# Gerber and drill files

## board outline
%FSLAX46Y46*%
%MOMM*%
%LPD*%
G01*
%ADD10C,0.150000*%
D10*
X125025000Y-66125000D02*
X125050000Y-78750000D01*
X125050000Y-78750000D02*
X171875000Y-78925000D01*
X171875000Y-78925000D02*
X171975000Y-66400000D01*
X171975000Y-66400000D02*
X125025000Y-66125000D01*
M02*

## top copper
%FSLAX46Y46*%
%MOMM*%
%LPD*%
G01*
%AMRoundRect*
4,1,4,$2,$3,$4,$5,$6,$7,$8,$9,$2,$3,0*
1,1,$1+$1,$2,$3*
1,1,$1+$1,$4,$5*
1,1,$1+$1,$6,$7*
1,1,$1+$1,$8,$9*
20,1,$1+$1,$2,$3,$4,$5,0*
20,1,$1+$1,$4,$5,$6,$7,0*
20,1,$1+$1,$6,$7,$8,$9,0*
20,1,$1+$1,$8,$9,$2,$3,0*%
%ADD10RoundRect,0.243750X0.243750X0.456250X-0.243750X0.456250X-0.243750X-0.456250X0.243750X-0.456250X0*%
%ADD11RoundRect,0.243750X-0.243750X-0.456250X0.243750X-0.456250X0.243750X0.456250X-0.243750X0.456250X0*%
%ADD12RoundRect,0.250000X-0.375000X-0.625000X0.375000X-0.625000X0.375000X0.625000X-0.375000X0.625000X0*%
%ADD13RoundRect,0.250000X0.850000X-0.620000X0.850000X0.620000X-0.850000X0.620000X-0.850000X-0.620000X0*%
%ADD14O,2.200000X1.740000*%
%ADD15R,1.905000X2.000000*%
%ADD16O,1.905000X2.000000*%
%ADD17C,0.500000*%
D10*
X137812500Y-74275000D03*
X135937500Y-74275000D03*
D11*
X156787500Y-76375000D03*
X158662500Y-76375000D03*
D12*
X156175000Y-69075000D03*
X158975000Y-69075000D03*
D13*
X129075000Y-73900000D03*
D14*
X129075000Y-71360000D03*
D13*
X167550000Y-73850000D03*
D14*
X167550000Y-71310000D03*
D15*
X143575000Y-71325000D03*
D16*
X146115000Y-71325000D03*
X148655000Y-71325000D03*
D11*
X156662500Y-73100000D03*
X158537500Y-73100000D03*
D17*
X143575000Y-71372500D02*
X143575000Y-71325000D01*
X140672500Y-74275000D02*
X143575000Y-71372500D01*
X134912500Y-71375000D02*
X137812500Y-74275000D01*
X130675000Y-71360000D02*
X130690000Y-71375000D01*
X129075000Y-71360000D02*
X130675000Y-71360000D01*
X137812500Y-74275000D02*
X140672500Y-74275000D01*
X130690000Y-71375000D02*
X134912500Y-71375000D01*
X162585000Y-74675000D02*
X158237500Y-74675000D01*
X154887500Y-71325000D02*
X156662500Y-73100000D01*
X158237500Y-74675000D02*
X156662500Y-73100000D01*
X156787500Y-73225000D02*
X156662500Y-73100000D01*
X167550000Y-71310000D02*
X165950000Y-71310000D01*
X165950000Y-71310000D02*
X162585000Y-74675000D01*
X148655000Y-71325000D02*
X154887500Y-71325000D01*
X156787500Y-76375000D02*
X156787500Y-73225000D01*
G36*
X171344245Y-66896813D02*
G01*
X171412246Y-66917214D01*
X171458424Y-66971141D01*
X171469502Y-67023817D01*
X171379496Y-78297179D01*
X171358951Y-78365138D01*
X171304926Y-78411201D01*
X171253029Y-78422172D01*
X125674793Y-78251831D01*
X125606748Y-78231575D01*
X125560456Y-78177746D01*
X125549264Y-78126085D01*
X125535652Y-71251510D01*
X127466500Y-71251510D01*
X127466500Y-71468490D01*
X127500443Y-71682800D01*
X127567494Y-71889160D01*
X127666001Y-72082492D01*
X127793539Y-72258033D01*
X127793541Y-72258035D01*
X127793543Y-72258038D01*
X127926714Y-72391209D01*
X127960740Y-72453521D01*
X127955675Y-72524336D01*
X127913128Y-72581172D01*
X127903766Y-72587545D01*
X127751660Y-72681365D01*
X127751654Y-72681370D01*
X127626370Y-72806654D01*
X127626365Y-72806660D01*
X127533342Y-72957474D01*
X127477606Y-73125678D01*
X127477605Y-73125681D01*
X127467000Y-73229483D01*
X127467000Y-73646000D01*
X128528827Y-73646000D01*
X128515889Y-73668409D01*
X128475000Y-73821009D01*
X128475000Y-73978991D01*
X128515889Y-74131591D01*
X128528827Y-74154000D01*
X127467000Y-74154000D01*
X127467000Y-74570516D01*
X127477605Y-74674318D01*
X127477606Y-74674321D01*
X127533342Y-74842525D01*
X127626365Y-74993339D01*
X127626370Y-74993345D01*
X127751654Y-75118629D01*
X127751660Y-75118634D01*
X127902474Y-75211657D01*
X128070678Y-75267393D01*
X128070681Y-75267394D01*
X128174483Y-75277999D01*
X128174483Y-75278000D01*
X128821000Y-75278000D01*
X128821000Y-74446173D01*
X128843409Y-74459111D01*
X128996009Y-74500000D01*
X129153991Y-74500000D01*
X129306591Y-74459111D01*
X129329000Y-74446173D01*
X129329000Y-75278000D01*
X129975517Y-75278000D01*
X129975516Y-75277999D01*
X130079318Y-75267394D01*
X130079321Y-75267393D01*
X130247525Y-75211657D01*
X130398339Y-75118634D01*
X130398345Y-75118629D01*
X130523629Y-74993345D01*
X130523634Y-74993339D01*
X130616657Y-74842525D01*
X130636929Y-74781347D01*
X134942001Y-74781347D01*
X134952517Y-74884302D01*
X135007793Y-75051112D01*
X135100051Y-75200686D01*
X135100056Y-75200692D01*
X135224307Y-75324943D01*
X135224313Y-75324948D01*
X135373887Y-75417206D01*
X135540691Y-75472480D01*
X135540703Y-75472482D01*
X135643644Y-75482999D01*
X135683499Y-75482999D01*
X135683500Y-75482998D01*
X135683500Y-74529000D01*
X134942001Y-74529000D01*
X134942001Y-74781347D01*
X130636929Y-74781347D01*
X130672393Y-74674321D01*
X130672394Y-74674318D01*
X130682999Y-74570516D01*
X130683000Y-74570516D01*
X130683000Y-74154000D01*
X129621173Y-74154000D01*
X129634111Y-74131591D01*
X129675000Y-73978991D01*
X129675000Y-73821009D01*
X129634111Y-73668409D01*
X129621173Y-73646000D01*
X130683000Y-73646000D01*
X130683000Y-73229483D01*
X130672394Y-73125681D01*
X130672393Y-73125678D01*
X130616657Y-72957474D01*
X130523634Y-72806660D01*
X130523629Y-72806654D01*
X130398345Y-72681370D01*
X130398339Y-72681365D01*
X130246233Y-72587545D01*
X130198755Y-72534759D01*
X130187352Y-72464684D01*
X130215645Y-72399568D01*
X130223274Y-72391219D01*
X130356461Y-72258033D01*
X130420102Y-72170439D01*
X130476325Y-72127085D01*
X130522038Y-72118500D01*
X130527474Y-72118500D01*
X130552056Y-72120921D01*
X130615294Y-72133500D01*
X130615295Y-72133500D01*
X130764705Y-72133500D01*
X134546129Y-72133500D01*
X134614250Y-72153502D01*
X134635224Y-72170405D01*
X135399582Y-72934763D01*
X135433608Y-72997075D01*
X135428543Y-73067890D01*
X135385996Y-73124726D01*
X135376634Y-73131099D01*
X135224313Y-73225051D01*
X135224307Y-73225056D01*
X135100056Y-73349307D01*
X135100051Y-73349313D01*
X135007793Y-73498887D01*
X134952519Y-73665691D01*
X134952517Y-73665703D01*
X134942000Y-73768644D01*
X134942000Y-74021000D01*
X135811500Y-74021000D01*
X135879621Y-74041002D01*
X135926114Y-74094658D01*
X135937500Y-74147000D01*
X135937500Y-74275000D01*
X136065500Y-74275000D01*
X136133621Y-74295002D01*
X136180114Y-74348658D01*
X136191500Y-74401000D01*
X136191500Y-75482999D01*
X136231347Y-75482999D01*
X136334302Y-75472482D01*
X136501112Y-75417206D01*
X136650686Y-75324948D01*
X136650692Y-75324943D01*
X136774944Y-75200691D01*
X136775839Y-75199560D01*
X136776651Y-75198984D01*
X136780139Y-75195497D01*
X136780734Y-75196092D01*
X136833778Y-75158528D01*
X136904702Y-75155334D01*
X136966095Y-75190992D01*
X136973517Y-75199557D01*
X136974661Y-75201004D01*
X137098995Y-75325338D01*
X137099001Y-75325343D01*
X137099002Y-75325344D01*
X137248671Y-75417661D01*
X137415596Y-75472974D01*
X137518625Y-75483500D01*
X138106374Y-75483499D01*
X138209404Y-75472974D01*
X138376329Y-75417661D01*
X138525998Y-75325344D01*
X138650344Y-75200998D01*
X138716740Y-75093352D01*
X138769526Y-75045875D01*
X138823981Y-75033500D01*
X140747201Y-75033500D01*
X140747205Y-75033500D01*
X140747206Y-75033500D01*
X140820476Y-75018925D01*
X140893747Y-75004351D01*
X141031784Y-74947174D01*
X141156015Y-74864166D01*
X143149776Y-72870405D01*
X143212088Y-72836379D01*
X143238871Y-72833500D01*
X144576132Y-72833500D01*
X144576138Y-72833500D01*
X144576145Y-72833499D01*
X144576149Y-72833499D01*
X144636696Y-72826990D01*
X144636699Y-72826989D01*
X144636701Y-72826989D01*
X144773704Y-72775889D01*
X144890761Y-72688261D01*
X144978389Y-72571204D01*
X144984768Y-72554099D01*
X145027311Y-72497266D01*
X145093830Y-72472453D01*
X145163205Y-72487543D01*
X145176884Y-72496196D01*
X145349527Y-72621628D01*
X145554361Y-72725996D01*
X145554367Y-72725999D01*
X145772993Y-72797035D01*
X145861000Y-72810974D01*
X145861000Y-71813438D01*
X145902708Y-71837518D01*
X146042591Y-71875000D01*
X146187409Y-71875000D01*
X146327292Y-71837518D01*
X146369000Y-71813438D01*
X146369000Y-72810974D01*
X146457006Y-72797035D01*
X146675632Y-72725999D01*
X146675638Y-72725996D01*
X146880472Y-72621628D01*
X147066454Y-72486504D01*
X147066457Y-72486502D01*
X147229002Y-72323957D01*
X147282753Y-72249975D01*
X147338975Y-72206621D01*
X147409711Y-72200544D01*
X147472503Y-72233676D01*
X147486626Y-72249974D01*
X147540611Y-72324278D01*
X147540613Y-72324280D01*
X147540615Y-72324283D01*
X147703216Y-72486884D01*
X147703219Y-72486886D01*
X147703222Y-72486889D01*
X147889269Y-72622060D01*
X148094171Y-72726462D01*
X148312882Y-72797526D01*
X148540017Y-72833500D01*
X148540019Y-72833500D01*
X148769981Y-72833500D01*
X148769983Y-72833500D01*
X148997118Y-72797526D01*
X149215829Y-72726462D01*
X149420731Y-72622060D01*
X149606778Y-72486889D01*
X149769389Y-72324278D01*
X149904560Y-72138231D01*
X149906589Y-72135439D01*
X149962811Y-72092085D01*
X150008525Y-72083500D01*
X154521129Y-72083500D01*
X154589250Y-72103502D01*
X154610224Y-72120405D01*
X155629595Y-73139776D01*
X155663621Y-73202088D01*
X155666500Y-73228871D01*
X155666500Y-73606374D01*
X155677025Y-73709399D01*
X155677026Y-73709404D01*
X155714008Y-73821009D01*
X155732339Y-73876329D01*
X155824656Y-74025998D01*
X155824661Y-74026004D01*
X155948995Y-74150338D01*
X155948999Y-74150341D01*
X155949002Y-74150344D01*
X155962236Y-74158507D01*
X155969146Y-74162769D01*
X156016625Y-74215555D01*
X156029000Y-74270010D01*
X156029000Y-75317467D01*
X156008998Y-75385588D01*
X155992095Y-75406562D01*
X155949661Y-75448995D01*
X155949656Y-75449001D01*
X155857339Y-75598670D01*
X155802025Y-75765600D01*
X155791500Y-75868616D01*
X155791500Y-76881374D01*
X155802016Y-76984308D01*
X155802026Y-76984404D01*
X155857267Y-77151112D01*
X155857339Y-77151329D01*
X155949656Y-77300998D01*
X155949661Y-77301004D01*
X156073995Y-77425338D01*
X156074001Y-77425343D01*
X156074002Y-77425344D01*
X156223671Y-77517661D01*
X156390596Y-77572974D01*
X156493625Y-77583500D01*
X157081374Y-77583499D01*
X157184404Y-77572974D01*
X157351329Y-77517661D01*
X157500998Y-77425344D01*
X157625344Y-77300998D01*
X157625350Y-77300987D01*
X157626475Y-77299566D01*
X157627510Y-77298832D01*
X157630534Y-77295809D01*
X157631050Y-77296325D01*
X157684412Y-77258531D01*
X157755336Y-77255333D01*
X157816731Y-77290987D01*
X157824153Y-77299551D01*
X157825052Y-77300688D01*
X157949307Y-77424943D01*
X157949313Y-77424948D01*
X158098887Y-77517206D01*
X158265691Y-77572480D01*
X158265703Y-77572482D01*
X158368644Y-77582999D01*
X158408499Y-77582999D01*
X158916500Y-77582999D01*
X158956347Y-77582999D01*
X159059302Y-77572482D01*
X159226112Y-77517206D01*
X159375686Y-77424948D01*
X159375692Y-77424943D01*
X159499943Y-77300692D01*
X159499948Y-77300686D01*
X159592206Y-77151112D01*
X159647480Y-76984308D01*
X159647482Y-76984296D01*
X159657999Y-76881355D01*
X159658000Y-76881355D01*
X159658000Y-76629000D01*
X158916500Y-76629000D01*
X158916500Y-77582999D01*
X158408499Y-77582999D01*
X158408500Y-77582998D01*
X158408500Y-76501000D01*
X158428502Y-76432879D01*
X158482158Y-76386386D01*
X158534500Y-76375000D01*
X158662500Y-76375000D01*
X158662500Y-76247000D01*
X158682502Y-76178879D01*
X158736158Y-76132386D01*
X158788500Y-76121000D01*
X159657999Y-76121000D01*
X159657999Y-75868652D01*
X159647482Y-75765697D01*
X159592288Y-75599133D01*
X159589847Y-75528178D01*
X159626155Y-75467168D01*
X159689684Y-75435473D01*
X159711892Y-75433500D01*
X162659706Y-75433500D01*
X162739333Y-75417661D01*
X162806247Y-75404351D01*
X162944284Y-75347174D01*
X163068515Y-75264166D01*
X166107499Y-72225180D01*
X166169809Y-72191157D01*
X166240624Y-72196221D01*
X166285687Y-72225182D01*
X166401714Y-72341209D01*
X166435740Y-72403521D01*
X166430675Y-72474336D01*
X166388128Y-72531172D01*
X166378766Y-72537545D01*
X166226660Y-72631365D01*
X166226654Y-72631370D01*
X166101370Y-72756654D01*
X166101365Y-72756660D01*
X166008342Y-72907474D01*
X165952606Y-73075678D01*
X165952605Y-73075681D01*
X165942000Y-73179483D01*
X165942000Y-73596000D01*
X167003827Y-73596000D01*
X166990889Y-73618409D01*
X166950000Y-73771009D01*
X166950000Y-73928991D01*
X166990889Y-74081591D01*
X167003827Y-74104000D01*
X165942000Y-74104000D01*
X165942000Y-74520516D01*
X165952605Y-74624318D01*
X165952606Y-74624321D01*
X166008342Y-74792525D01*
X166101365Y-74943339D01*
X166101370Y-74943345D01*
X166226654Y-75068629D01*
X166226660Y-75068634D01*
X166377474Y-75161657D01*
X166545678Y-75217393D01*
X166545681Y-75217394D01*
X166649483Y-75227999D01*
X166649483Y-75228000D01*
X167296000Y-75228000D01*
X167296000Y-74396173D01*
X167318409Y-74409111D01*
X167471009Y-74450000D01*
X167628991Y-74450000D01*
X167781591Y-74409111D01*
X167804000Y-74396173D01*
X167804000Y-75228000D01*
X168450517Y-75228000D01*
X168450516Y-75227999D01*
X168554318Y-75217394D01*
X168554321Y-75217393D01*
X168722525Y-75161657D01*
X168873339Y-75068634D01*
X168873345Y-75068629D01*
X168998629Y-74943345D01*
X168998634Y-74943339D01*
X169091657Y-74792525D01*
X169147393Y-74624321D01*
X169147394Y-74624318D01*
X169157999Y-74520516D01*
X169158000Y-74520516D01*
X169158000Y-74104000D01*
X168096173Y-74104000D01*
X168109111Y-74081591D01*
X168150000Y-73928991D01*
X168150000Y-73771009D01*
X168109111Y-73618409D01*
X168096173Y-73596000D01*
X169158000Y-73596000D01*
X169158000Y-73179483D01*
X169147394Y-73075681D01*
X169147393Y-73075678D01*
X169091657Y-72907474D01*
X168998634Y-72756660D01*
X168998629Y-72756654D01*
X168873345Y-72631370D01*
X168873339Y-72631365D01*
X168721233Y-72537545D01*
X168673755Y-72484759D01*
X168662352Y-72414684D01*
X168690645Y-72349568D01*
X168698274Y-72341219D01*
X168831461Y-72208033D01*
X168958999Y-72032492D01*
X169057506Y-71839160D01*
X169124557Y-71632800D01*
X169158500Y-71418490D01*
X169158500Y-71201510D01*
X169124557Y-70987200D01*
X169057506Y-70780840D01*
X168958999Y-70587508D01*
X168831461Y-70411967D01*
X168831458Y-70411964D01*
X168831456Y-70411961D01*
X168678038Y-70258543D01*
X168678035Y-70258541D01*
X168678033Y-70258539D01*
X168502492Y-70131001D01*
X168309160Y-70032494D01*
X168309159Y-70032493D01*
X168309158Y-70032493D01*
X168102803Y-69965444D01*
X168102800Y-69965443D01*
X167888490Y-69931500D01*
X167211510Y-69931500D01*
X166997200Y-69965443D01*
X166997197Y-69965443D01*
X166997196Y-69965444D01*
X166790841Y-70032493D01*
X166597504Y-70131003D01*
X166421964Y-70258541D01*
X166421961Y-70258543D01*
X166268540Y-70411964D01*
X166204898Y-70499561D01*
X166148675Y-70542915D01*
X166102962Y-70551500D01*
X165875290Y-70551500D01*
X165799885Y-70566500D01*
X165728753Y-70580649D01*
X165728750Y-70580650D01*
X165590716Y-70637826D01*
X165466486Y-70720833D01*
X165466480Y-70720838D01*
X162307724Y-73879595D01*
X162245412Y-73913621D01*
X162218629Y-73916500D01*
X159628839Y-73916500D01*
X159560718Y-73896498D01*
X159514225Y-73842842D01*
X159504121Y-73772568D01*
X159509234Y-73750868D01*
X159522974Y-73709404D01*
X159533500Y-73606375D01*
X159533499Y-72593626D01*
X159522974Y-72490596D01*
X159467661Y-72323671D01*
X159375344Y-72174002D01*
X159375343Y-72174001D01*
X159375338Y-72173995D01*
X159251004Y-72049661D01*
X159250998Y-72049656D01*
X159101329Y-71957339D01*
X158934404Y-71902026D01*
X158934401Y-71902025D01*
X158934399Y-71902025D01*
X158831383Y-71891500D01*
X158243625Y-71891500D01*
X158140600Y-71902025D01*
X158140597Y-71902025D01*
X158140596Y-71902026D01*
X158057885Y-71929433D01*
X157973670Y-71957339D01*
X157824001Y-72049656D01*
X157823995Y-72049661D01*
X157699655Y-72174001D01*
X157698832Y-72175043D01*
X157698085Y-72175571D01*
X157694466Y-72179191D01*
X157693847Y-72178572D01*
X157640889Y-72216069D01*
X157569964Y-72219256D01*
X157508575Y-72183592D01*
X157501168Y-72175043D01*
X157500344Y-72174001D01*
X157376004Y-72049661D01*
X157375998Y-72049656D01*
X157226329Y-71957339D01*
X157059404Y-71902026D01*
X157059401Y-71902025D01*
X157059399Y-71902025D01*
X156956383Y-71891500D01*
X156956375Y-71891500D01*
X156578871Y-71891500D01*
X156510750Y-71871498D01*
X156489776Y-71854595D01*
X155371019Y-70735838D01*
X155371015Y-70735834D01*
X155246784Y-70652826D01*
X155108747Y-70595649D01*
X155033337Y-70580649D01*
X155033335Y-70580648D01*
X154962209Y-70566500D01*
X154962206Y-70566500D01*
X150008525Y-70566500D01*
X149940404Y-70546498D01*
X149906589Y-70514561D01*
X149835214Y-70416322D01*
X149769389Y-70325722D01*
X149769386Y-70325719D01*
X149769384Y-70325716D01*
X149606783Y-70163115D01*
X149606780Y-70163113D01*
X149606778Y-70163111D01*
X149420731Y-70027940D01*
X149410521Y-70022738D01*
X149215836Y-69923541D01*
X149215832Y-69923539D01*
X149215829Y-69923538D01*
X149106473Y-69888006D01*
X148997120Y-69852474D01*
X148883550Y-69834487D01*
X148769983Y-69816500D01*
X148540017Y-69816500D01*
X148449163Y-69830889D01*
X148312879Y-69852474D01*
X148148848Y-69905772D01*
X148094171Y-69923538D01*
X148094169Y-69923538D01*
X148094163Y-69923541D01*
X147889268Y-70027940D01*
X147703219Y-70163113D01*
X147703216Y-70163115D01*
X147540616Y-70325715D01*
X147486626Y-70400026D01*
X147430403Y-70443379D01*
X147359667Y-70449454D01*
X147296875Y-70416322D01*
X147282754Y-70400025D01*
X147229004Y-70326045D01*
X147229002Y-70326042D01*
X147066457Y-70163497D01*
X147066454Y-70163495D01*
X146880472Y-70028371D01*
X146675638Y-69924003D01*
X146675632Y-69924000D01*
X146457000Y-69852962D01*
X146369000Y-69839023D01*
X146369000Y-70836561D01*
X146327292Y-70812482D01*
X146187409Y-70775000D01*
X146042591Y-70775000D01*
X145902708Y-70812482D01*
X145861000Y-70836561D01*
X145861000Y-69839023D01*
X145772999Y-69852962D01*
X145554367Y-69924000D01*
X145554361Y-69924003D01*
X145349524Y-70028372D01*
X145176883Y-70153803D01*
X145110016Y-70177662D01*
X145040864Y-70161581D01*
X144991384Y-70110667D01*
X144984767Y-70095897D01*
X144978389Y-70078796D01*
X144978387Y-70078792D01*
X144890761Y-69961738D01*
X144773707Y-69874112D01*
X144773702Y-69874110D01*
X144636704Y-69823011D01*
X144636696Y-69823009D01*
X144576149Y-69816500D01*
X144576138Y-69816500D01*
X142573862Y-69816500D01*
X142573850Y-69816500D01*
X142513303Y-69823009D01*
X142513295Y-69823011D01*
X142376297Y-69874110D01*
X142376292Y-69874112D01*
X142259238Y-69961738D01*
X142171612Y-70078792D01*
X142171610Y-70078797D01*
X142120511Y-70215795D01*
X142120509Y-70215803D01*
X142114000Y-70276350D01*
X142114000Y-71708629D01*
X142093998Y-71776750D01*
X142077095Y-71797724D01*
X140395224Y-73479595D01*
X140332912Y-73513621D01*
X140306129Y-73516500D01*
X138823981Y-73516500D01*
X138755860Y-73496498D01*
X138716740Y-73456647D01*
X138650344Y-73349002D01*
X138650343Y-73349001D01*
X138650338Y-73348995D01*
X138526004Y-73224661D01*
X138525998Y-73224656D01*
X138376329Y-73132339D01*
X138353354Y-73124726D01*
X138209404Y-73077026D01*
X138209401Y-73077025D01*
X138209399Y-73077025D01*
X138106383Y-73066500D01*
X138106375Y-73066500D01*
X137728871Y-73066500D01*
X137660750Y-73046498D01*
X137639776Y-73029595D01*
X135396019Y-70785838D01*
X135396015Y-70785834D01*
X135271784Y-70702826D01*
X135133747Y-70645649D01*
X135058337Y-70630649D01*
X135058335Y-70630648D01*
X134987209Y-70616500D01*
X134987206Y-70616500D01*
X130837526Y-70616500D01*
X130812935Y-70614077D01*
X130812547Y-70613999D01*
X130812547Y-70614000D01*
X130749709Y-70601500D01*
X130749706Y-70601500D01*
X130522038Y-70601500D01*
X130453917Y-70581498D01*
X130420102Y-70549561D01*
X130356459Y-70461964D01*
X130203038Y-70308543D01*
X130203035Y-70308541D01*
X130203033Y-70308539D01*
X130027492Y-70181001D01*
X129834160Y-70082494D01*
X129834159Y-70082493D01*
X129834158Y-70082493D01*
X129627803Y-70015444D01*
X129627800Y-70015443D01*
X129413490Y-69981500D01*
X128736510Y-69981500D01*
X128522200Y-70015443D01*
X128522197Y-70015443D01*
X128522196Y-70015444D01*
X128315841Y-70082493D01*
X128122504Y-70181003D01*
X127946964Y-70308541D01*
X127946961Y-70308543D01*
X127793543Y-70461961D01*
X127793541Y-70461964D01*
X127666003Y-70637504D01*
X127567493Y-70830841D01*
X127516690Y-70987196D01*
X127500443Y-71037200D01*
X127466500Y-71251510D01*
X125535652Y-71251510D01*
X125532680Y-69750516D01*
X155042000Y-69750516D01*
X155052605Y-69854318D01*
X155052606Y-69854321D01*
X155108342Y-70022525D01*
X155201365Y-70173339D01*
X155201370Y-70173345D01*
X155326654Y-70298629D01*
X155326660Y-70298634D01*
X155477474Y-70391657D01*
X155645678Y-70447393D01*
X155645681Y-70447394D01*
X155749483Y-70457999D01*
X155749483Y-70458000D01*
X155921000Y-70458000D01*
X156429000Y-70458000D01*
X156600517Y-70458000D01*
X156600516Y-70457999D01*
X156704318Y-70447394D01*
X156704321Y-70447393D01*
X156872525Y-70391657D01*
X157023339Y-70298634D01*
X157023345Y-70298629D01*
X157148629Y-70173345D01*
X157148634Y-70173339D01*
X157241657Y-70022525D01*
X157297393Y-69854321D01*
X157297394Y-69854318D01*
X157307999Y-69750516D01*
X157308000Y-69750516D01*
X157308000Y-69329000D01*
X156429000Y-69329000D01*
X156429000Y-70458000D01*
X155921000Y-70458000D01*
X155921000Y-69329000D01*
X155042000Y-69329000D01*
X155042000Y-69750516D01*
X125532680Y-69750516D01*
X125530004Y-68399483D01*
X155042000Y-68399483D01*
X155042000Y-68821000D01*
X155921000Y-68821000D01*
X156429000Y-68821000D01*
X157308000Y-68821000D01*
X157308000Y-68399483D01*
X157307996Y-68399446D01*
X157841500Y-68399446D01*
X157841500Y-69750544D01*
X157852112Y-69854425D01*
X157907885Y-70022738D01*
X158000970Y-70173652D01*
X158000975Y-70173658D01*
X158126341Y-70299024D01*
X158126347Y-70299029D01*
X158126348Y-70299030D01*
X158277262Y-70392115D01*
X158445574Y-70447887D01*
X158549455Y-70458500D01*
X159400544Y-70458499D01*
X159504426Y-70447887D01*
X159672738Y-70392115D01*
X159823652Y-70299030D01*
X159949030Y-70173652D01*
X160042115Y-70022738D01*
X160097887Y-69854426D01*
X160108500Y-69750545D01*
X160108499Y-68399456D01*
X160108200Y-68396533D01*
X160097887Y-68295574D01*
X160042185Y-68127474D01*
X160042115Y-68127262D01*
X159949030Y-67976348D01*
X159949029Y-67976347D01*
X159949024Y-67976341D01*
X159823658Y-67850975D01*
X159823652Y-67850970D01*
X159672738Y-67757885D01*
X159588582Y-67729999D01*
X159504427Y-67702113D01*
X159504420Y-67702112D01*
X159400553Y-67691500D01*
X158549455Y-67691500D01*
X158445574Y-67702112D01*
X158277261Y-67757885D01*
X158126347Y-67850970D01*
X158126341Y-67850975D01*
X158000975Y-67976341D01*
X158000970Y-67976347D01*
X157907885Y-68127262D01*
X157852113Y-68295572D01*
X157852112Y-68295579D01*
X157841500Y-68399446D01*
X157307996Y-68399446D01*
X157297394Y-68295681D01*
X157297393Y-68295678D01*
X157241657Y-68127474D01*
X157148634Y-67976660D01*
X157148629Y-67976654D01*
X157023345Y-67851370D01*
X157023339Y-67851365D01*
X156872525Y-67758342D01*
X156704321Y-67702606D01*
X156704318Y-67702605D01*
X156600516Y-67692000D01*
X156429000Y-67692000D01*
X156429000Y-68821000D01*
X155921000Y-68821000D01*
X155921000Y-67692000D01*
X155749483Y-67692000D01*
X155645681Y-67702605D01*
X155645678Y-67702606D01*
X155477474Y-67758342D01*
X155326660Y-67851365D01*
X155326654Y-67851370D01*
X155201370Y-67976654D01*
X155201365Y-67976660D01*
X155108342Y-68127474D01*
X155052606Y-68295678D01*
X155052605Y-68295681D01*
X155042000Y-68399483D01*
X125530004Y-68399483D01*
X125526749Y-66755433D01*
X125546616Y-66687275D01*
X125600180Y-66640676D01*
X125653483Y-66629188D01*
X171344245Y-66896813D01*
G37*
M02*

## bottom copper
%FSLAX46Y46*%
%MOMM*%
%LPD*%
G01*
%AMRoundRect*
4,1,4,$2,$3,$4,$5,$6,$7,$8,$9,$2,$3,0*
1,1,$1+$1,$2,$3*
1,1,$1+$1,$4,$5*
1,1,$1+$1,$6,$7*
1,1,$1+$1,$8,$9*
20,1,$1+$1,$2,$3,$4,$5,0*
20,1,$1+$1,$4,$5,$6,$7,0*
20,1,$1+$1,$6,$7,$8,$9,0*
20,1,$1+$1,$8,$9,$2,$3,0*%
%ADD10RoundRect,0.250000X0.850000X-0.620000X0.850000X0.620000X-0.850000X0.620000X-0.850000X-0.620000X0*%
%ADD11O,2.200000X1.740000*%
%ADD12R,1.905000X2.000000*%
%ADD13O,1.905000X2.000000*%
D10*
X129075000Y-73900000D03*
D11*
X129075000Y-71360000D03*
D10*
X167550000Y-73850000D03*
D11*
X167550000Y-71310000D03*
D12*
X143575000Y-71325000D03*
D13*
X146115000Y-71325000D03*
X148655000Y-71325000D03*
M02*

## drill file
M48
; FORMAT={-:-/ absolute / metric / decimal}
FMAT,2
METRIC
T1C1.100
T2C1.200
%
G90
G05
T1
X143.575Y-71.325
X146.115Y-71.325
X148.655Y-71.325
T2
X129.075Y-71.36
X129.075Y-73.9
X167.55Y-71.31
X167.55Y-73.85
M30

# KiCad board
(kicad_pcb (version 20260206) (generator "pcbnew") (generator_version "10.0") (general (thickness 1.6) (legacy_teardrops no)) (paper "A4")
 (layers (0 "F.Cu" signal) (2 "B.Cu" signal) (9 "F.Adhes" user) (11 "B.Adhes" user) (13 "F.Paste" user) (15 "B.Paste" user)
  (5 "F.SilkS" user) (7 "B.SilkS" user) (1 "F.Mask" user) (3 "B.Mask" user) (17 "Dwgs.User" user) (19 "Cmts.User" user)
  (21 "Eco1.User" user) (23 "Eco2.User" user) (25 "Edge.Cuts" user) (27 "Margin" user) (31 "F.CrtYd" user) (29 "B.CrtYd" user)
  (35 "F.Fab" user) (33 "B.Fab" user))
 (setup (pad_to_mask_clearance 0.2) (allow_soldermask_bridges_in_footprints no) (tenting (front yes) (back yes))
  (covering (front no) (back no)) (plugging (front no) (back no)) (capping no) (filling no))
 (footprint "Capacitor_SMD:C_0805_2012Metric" (layer "F.Cu") (at 136.875 74.275 180)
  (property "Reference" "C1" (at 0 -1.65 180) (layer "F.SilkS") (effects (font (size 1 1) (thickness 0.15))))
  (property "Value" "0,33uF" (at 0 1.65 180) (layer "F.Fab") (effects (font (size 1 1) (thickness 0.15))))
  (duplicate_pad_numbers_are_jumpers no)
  (pad "1" smd roundrect (at -0.9375 0 180) (size 0.975 1.4) (layers "F.Cu" "F.Mask" "F.Paste") (roundrect_rratio 0.25)
   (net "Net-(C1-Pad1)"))
  (pad "2" smd roundrect (at 0.9375 0 180) (size 0.975 1.4) (layers "F.Cu" "F.Mask" "F.Paste") (roundrect_rratio 0.25) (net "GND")))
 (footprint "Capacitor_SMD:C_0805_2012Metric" (layer "F.Cu") (at 157.725 76.375)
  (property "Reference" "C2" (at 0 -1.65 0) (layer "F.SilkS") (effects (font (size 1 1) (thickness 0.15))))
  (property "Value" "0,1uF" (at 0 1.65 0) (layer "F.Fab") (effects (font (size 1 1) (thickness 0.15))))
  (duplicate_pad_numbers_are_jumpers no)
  (pad "1" smd roundrect (at -0.9375 0) (size 0.975 1.4) (layers "F.Cu" "F.Mask" "F.Paste") (roundrect_rratio 0.25) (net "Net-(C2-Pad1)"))
  (pad "2" smd roundrect (at 0.9375 0) (size 0.975 1.4) (layers "F.Cu" "F.Mask" "F.Paste") (roundrect_rratio 0.25) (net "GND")))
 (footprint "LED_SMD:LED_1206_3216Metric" (layer "F.Cu") (at 157.575 69.075)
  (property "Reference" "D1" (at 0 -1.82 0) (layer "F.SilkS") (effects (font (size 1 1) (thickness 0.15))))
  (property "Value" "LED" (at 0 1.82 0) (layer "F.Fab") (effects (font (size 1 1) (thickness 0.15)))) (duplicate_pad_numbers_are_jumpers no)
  (pad "1" smd roundrect (at -1.4 0) (size 1.25 1.75) (layers "F.Cu" "F.Mask" "F.Paste") (roundrect_rratio 0.2) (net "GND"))
  (pad "2" smd roundrect (at 1.4 0) (size 1.25 1.75) (layers "F.Cu" "F.Mask" "F.Paste") (roundrect_rratio 0.2) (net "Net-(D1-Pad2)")))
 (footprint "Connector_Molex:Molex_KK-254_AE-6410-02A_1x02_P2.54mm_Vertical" (layer "F.Cu") (at 129.075 73.9 90)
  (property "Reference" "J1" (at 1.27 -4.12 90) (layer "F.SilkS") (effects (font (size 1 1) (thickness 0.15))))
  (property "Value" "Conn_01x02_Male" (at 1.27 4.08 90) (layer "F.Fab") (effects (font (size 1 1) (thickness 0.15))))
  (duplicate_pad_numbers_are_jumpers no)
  (pad "1" thru_hole roundrect (at 0 0 90) (size 1.74 2.2) (drill 1.2) (layers "*.Cu" "*.Mask") (remove_unused_layers no)
   (roundrect_rratio 0.143678) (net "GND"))
  (pad "2" thru_hole oval (at 2.54 0 90) (size 1.74 2.2) (drill 1.2) (layers "*.Cu" "*.Mask") (remove_unused_layers no)
   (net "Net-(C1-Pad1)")))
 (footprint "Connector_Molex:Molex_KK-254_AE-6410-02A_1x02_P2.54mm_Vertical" (layer "F.Cu") (at 167.55 73.85 90)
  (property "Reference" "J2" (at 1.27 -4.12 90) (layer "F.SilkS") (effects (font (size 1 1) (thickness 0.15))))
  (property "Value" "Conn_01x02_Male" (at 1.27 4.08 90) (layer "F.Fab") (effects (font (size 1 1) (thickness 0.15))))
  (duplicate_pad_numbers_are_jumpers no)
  (pad "1" thru_hole roundrect (at 0 0 90) (size 1.74 2.2) (drill 1.2) (layers "*.Cu" "*.Mask") (remove_unused_layers no)
   (roundrect_rratio 0.143678) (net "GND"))
  (pad "2" thru_hole oval (at 2.54 0 90) (size 1.74 2.2) (drill 1.2) (layers "*.Cu" "*.Mask") (remove_unused_layers no)
   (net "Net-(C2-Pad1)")))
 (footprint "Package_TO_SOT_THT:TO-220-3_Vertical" (layer "F.Cu") (at 143.575 71.325)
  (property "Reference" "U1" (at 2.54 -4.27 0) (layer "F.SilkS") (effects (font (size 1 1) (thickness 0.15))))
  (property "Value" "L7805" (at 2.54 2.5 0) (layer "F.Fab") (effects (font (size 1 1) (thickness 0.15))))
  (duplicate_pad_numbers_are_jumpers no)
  (pad "1" thru_hole rect (at 0 0) (size 1.905 2) (drill 1.1) (layers "*.Cu" "*.Mask") (remove_unused_layers no) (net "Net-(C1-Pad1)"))
  (pad "2" thru_hole oval (at 2.54 0) (size 1.905 2) (drill 1.1) (layers "*.Cu" "*.Mask") (remove_unused_layers no) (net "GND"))
  (pad "3" thru_hole oval (at 5.08 0) (size 1.905 2) (drill 1.1) (layers "*.Cu" "*.Mask") (remove_unused_layers no) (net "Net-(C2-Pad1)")))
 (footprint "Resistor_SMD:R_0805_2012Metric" (layer "F.Cu") (at 157.6 73.1)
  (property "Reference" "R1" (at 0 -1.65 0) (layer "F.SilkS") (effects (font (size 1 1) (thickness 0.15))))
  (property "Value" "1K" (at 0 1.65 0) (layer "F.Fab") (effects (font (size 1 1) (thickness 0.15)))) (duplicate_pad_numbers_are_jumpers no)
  (pad "1" smd roundrect (at -0.9375 0) (size 0.975 1.4) (layers "F.Cu" "F.Mask" "F.Paste") (roundrect_rratio 0.25) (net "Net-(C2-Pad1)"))
  (pad "2" smd roundrect (at 0.9375 0) (size 0.975 1.4) (layers "F.Cu" "F.Mask" "F.Paste") (roundrect_rratio 0.25) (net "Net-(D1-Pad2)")))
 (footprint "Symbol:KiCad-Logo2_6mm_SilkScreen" (layer "B.Cu") (at 157.63 71.98 180)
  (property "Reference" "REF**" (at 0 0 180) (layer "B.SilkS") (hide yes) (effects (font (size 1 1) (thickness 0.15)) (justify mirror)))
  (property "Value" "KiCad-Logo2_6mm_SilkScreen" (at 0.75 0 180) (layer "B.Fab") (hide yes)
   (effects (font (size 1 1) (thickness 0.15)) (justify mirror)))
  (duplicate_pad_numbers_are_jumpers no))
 (gr_line (start 125.025 66.125) (end 125.05 78.75) (stroke (width 0.15) (type solid)) (layer "Edge.Cuts"))
 (gr_line (start 125.05 78.75) (end 171.875 78.925) (stroke (width 0.15) (type solid)) (layer "Edge.Cuts"))
 (gr_line (start 171.875 78.925) (end 171.975 66.4) (stroke (width 0.15) (type solid)) (layer "Edge.Cuts"))
 (gr_line (start 171.975 66.4) (end 125.025 66.125) (stroke (width 0.15) (type solid)) (layer "Edge.Cuts"))
 (segment (start 143.575 71.3725) (end 143.575 71.325) (width 0.5) (layer "F.Cu") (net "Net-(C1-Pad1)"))
 (segment (start 140.6725 74.275) (end 143.575 71.3725) (width 0.5) (layer "F.Cu") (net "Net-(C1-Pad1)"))
 (segment (start 134.9125 71.375) (end 137.8125 74.275) (width 0.5) (layer "F.Cu") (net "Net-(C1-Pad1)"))
 (segment (start 130.675 71.36) (end 130.69 71.375) (width 0.5) (layer "F.Cu") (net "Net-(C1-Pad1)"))
 (segment (start 129.075 71.36) (end 130.675 71.36) (width 0.5) (layer "F.Cu") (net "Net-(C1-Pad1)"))
 (segment (start 137.8125 74.275) (end 140.6725 74.275) (width 0.5) (layer "F.Cu") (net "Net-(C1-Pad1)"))
 (segment (start 130.69 71.375) (end 134.9125 71.375) (width 0.5) (layer "F.Cu") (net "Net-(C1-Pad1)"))
 (segment (start 162.585 74.675) (end 158.2375 74.675) (width 0.5) (layer "F.Cu") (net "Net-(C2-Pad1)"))
 (segment (start 154.8875 71.325) (end 156.6625 73.1) (width 0.5) (layer "F.Cu") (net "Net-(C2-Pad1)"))
 (segment (start 158.2375 74.675) (end 156.6625 73.1) (width 0.5) (layer "F.Cu") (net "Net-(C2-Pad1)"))
 (segment (start 156.7875 73.225) (end 156.6625 73.1) (width 0.5) (layer "F.Cu") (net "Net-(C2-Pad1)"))
 (segment (start 167.55 71.31) (end 165.95 71.31) (width 0.5) (layer "F.Cu") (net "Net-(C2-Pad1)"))
 (segment (start 165.95 71.31) (end 162.585 74.675) (width 0.5) (layer "F.Cu") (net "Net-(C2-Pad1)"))
 (segment (start 148.655 71.325) (end 154.8875 71.325) (width 0.5) (layer "F.Cu") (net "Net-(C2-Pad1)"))
 (segment (start 156.7875 76.375) (end 156.7875 73.225) (width 0.5) (layer "F.Cu") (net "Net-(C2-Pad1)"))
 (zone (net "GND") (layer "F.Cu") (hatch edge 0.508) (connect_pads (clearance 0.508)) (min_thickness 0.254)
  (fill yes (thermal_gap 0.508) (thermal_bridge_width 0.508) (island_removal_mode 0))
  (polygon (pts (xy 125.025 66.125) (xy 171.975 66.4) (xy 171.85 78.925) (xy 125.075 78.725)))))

